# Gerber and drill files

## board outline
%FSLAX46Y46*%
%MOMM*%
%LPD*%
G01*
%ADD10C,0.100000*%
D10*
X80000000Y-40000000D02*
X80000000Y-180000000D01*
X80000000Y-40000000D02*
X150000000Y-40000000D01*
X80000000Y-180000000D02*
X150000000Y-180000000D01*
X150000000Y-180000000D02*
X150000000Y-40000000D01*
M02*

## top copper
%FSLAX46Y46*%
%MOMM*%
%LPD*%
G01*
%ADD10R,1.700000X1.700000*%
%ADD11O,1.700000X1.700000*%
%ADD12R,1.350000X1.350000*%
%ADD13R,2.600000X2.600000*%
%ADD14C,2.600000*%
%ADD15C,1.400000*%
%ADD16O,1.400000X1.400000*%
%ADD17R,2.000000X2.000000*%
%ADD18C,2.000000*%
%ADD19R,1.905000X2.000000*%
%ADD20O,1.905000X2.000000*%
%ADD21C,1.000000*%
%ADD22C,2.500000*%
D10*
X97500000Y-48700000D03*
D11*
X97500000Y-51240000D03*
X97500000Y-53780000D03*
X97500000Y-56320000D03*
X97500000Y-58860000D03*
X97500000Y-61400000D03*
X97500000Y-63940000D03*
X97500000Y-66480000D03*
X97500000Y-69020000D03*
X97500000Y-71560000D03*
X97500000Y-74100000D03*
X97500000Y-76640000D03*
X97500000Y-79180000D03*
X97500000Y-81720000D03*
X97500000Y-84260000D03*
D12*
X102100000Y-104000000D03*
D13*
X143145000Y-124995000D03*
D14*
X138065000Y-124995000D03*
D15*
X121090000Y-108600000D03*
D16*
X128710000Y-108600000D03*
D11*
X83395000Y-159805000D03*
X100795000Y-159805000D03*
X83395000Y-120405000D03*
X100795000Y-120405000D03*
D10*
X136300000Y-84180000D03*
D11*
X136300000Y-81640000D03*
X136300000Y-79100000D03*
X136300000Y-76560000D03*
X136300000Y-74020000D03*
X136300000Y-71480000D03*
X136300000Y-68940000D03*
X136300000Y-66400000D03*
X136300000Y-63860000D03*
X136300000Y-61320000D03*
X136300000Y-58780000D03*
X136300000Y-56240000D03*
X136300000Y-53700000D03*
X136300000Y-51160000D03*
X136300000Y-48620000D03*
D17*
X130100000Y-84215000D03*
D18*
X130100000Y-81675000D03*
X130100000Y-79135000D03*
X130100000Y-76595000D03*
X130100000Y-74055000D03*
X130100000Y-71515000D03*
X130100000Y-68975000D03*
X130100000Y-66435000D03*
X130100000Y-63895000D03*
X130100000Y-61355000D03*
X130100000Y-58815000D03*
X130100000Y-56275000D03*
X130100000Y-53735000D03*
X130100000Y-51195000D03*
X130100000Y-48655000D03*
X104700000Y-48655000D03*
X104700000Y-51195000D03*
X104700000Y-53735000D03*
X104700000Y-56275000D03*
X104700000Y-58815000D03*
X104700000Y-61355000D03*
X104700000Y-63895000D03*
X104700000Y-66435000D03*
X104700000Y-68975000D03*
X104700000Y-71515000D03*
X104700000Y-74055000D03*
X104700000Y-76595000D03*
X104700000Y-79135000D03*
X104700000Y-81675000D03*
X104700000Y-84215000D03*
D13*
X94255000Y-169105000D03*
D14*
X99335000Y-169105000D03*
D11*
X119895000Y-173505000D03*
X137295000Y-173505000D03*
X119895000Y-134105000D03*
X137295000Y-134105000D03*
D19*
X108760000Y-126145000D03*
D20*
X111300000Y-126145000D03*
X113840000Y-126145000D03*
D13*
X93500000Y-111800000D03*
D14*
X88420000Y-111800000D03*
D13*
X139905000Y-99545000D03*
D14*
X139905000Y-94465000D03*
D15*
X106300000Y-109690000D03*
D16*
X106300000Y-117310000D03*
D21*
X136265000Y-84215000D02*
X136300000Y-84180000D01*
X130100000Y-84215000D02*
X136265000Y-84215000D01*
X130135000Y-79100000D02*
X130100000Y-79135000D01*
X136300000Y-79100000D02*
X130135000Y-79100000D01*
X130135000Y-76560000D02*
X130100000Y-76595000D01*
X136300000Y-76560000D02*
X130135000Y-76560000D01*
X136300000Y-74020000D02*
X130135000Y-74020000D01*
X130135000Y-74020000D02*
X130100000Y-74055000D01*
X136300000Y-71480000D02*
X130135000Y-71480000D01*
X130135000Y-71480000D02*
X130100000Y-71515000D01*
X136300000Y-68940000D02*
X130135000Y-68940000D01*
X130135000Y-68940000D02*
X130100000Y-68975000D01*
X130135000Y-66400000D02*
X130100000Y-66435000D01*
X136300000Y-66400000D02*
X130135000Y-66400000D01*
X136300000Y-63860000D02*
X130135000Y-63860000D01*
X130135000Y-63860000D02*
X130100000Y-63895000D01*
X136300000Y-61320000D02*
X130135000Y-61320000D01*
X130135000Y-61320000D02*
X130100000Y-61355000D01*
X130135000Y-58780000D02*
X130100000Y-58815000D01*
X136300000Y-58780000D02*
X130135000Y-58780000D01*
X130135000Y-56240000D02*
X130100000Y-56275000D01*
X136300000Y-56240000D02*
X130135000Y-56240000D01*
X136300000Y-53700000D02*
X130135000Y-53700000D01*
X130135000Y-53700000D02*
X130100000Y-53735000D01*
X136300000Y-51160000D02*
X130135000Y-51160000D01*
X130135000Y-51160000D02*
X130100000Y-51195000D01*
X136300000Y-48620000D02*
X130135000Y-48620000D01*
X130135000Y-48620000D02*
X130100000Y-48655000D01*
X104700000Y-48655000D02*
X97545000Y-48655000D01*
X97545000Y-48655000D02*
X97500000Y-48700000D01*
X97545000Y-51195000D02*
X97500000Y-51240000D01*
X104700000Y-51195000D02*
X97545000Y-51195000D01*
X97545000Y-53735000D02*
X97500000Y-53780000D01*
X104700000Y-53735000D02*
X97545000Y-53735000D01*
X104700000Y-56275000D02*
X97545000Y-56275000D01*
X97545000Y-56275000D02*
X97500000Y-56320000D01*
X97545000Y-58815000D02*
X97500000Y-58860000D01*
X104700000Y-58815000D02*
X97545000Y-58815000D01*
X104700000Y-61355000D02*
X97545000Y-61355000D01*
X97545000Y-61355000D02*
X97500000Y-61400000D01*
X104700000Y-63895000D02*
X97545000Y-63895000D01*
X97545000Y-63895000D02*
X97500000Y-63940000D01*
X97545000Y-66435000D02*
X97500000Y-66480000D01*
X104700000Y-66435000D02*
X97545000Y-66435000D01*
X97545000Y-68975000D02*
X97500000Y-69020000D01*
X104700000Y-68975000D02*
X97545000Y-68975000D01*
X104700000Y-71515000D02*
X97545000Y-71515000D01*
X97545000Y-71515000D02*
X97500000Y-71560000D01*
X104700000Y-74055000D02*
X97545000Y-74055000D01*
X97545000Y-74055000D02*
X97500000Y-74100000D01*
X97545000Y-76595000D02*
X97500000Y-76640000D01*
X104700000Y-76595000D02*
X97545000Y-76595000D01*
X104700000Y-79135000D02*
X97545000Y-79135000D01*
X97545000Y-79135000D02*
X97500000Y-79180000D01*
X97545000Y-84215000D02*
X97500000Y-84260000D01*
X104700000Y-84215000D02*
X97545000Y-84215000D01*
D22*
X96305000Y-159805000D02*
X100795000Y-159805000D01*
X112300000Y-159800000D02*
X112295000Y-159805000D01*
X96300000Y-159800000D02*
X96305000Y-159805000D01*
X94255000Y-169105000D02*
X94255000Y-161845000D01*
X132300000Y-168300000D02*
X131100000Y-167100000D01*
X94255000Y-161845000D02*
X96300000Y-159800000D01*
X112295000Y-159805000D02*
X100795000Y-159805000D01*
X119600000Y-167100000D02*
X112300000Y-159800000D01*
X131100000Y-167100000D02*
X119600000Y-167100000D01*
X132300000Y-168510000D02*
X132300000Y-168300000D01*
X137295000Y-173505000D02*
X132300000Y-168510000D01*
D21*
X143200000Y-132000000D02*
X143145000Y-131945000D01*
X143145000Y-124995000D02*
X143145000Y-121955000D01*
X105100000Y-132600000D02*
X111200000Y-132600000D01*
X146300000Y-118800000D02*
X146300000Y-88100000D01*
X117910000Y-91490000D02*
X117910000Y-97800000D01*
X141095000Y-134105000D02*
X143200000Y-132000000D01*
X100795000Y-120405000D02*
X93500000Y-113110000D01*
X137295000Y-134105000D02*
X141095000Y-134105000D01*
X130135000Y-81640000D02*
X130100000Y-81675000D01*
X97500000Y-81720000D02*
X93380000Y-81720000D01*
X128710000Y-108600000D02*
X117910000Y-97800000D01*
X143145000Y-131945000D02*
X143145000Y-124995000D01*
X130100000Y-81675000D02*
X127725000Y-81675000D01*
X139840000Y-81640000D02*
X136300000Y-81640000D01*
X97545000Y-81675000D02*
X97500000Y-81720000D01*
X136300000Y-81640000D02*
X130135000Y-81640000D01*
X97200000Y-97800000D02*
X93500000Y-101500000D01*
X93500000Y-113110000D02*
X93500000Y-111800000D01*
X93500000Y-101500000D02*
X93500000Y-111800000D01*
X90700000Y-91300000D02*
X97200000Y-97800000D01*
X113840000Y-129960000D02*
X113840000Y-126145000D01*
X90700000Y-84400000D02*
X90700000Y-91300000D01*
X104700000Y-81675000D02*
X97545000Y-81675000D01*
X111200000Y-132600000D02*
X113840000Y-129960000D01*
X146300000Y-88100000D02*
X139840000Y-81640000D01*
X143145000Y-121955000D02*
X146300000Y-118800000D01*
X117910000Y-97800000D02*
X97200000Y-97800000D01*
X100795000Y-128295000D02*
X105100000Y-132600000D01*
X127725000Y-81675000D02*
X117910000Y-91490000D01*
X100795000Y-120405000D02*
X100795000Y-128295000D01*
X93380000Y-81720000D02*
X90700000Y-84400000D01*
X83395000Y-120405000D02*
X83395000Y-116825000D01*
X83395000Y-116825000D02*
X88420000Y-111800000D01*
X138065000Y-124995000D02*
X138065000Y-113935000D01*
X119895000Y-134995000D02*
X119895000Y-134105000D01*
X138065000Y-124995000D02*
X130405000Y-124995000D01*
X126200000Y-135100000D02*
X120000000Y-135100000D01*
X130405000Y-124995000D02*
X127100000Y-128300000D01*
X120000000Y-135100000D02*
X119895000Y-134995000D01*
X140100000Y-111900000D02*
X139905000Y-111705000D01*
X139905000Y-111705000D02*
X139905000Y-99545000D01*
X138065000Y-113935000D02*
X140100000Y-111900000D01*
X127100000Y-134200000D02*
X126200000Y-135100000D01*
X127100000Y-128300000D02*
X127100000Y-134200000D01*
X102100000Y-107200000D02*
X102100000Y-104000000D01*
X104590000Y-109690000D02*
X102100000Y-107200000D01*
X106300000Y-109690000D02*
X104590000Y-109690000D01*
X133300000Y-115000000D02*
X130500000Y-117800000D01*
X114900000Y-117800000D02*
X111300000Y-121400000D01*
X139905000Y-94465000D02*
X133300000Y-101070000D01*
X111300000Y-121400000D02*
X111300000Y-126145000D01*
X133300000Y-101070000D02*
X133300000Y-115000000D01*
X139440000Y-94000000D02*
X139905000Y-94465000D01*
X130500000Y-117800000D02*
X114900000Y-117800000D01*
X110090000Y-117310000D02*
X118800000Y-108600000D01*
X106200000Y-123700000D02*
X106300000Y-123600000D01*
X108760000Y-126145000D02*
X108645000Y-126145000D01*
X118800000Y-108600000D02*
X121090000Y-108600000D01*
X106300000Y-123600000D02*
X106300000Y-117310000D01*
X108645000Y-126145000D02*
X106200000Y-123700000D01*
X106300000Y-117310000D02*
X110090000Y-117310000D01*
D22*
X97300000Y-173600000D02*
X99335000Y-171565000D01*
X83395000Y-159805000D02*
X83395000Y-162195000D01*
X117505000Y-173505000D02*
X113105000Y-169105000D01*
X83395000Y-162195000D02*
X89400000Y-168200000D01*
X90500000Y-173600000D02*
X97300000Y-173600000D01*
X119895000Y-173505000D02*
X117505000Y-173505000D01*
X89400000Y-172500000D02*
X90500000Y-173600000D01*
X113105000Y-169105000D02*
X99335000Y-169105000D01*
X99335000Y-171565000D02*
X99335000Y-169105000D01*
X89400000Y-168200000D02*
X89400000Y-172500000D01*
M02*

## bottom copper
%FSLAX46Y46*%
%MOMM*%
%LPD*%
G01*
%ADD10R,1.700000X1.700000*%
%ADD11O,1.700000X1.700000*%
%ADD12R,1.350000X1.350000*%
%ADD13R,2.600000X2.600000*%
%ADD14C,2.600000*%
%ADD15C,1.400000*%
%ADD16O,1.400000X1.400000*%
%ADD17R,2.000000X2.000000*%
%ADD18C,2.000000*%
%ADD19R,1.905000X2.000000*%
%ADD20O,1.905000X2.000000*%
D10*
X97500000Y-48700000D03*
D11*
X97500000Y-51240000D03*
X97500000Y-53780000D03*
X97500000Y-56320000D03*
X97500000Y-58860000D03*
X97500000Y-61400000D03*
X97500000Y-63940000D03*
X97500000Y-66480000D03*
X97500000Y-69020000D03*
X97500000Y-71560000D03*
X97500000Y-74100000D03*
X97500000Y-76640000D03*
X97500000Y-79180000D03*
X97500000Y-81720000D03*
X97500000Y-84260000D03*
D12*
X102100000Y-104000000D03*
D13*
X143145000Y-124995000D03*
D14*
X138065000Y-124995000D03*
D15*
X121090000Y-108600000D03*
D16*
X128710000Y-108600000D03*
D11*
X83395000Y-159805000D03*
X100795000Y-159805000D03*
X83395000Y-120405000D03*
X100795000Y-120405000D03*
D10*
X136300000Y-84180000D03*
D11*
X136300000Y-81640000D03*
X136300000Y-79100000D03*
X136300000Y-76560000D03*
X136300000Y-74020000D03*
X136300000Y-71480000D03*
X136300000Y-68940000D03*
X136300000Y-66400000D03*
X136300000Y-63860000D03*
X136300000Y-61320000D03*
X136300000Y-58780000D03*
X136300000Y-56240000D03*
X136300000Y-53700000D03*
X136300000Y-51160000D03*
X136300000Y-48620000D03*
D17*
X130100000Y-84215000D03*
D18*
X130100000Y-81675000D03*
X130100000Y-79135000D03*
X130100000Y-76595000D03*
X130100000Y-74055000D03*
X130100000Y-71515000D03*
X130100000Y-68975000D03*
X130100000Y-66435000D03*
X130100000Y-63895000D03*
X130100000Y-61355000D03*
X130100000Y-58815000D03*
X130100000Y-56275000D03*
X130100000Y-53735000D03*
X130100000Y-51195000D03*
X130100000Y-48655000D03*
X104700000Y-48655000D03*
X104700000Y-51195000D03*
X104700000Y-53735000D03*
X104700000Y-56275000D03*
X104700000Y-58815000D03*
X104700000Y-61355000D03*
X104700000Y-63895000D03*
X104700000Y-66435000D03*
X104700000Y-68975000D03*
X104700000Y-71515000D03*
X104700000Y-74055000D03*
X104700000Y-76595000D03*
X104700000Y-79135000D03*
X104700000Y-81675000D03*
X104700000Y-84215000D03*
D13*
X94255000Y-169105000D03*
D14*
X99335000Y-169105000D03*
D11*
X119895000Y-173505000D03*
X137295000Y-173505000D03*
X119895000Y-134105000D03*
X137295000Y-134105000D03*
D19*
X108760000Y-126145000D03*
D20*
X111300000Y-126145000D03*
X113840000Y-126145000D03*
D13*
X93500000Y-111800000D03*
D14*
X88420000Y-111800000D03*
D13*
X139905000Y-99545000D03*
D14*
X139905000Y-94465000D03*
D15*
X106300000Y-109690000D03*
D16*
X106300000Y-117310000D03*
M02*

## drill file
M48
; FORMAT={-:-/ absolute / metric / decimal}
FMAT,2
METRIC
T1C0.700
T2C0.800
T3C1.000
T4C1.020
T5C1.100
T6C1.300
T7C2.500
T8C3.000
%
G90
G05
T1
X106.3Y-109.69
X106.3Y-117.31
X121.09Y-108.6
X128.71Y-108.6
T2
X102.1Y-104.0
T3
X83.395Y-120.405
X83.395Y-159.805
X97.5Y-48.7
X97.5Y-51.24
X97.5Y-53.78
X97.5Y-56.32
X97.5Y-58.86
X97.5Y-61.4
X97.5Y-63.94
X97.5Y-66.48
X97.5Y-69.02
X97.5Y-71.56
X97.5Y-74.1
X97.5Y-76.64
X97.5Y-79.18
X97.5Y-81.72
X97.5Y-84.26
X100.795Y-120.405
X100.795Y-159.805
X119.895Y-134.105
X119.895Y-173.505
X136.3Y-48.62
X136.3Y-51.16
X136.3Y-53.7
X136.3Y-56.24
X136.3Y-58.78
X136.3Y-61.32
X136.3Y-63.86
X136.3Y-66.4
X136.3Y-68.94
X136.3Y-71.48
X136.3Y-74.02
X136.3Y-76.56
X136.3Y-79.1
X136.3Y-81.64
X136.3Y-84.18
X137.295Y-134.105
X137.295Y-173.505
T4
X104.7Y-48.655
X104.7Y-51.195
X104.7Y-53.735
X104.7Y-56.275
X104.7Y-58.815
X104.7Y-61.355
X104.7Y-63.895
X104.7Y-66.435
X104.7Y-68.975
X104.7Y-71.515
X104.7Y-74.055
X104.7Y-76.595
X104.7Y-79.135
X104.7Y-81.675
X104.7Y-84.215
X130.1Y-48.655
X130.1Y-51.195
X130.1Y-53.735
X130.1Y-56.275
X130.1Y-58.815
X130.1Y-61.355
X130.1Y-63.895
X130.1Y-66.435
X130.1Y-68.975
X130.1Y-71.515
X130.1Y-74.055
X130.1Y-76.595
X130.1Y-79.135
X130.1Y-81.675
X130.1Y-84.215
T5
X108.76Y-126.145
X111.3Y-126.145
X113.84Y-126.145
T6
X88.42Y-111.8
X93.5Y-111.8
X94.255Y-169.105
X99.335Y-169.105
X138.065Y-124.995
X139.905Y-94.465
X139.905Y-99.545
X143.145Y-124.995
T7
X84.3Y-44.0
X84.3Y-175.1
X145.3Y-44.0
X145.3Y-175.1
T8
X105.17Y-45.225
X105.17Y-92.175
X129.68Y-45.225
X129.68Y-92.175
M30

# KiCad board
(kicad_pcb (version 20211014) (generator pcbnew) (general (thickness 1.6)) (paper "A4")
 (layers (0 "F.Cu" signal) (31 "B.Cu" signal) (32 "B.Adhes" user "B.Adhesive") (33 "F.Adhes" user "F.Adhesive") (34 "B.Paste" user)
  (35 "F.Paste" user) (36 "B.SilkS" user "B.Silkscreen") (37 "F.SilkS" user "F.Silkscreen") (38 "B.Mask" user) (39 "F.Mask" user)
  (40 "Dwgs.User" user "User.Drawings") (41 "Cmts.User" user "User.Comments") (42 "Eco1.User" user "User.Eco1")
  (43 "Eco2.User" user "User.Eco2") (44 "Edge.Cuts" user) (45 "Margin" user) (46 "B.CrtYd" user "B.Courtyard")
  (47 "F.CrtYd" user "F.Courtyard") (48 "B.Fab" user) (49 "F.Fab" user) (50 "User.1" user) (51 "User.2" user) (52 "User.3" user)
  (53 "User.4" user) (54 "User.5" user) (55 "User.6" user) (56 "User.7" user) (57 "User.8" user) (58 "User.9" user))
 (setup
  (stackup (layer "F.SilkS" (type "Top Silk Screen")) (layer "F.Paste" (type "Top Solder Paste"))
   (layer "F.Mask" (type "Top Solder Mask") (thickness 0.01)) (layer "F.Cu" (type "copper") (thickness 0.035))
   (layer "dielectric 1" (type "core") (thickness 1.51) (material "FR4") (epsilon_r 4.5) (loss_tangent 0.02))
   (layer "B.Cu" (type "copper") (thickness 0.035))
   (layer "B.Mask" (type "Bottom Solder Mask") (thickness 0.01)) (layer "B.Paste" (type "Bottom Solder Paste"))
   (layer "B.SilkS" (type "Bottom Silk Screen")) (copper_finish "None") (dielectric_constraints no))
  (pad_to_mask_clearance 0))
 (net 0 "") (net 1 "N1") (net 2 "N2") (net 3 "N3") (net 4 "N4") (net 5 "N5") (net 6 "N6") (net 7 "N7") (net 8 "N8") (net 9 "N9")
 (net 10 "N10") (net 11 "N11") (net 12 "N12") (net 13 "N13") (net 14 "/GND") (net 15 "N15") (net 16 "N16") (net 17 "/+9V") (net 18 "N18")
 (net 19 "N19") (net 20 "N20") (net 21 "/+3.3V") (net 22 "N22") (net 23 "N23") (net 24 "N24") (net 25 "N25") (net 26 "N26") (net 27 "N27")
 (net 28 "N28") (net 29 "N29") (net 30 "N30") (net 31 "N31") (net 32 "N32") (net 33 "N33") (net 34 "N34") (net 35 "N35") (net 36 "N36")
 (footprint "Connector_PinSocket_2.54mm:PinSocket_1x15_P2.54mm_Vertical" (layer "F.Cu") (at 97.5 48.7)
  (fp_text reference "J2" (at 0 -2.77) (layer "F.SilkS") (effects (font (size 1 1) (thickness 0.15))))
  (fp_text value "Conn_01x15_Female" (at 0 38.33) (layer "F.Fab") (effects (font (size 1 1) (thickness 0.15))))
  (pad "1" thru_hole rect (at 0 0) (size 1.7 1.7) (drill 1) (layers *.Cu *.Mask) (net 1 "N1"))
  (pad "2" thru_hole oval (at 0 2.54) (size 1.7 1.7) (drill 1) (layers *.Cu *.Mask) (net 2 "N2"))
  (pad "3" thru_hole oval (at 0 5.08) (size 1.7 1.7) (drill 1) (layers *.Cu *.Mask) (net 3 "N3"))
  (pad "4" thru_hole oval (at 0 7.62) (size 1.7 1.7) (drill 1) (layers *.Cu *.Mask) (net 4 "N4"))
  (pad "5" thru_hole oval (at 0 10.16) (size 1.7 1.7) (drill 1) (layers *.Cu *.Mask) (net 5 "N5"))
  (pad "6" thru_hole oval (at 0 12.7) (size 1.7 1.7) (drill 1) (layers *.Cu *.Mask) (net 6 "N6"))
  (pad "7" thru_hole oval (at 0 15.24) (size 1.7 1.7) (drill 1) (layers *.Cu *.Mask) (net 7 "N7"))
  (pad "8" thru_hole oval (at 0 17.78) (size 1.7 1.7) (drill 1) (layers *.Cu *.Mask) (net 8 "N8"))
  (pad "9" thru_hole oval (at 0 20.32) (size 1.7 1.7) (drill 1) (layers *.Cu *.Mask) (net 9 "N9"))
  (pad "10" thru_hole oval (at 0 22.86) (size 1.7 1.7) (drill 1) (layers *.Cu *.Mask) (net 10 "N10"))
  (pad "11" thru_hole oval (at 0 25.4) (size 1.7 1.7) (drill 1) (layers *.Cu *.Mask) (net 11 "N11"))
  (pad "12" thru_hole oval (at 0 27.94) (size 1.7 1.7) (drill 1) (layers *.Cu *.Mask) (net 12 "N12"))
  (pad "13" thru_hole oval (at 0 30.48) (size 1.7 1.7) (drill 1) (layers *.Cu *.Mask) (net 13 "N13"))
  (pad "14" thru_hole oval (at 0 33.02) (size 1.7 1.7) (drill 1) (layers *.Cu *.Mask) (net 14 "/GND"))
  (pad "15" thru_hole oval (at 0 35.56) (size 1.7 1.7) (drill 1) (layers *.Cu *.Mask) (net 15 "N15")))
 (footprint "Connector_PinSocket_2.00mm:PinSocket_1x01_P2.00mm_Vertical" (layer "F.Cu") (at 102.1 104)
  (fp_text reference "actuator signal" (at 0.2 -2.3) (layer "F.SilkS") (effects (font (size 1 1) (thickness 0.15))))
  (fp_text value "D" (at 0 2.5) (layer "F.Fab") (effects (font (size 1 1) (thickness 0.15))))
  (pad "1" thru_hole rect (at 0 0) (size 1.35 1.35) (drill 0.8) (layers *.Cu *.Mask) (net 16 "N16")))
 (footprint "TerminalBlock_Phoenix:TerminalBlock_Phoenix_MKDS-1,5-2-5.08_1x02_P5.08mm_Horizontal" (layer "F.Cu") (at 143.145 124.995 180)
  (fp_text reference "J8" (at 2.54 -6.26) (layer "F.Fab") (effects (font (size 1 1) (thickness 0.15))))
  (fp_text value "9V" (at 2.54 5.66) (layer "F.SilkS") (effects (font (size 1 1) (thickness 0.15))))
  (pad "1" thru_hole rect (at 0 0 180) (size 2.6 2.6) (drill 1.3) (layers *.Cu *.Mask) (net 14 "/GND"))
  (pad "2" thru_hole circle (at 5.08 0 180) (size 2.6 2.6) (drill 1.3) (layers *.Cu *.Mask) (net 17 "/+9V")))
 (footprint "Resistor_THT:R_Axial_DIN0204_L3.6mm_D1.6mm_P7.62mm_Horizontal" (layer "F.Cu") (at 121.09 108.6)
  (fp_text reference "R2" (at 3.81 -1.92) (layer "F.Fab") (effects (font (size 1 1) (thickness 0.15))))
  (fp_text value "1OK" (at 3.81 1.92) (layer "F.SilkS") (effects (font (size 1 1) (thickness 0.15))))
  (pad "1" thru_hole circle (at 0 0) (size 1.4 1.4) (drill 0.7) (layers *.Cu *.Mask) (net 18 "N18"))
  (pad "2" thru_hole oval (at 7.62 0) (size 1.4 1.4) (drill 0.7) (layers *.Cu *.Mask) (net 14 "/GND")))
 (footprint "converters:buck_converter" (layer "F.Cu") (at 81.595 161.805 90)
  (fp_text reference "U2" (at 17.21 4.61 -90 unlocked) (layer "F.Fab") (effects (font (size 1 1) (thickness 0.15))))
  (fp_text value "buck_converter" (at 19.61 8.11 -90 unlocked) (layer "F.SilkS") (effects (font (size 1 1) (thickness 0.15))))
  (pad "1" thru_hole oval (at 2 1.8 90) (size 1.7 1.7) (drill 1) (layers *.Cu *.Mask) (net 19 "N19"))
  (pad "2" thru_hole oval (at 2 19.2 90) (size 1.7 1.7) (drill 1) (layers *.Cu *.Mask) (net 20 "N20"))
  (pad "3" thru_hole oval (at 41.4 1.8 90) (size 1.7 1.7) (drill 1) (layers *.Cu *.Mask) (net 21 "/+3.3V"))
  (pad "4" thru_hole oval (at 41.4 19.2 90) (size 1.7 1.7) (drill 1) (layers *.Cu *.Mask) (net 14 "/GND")))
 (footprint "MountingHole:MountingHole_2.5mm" (layer "F.Cu") (at 145.3 44)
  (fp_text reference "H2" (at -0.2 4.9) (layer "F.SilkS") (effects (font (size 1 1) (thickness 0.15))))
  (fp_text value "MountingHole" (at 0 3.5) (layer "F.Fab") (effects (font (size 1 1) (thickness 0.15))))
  (pad "" np_thru_hole circle (at 0 0) (size 2.5 2.5) (drill 2.5) (layers *.Cu *.Mask)))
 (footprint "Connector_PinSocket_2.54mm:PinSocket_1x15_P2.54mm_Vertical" (layer "F.Cu") (at 136.3 84.18 180)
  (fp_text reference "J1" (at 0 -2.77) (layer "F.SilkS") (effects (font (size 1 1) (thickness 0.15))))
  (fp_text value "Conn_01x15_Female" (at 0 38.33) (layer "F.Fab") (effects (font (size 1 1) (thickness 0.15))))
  (pad "1" thru_hole rect (at 0 0 180) (size 1.7 1.7) (drill 1) (layers *.Cu *.Mask) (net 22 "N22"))
  (pad "2" thru_hole oval (at 0 2.54 180) (size 1.7 1.7) (drill 1) (layers *.Cu *.Mask) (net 14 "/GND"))
  (pad "3" thru_hole oval (at 0 5.08 180) (size 1.7 1.7) (drill 1) (layers *.Cu *.Mask) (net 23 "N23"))
  (pad "4" thru_hole oval (at 0 7.62 180) (size 1.7 1.7) (drill 1) (layers *.Cu *.Mask) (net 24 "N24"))
  (pad "5" thru_hole oval (at 0 10.16 180) (size 1.7 1.7) (drill 1) (layers *.Cu *.Mask) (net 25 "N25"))
  (pad "6" thru_hole oval (at 0 12.7 180) (size 1.7 1.7) (drill 1) (layers *.Cu *.Mask) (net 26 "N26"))
  (pad "7" thru_hole oval (at 0 15.24 180) (size 1.7 1.7) (drill 1) (layers *.Cu *.Mask) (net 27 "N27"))
  (pad "8" thru_hole oval (at 0 17.78 180) (size 1.7 1.7) (drill 1) (layers *.Cu *.Mask) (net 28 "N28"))
  (pad "9" thru_hole oval (at 0 20.32 180) (size 1.7 1.7) (drill 1) (layers *.Cu *.Mask) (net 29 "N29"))
  (pad "10" thru_hole oval (at 0 22.86 180) (size 1.7 1.7) (drill 1) (layers *.Cu *.Mask) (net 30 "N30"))
  (pad "11" thru_hole oval (at 0 25.4 180) (size 1.7 1.7) (drill 1) (layers *.Cu *.Mask) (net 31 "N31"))
  (pad "12" thru_hole oval (at 0 27.94 180) (size 1.7 1.7) (drill 1) (layers *.Cu *.Mask) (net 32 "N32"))
  (pad "13" thru_hole oval (at 0 30.48 180) (size 1.7 1.7) (drill 1) (layers *.Cu *.Mask) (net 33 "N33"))
  (pad "14" thru_hole oval (at 0 33.02 180) (size 1.7 1.7) (drill 1) (layers *.Cu *.Mask) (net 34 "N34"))
  (pad "15" thru_hole oval (at 0 35.56 180) (size 1.7 1.7) (drill 1) (layers *.Cu *.Mask) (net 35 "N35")))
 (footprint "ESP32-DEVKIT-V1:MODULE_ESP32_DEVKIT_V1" (layer "F.Cu") (at 117.4 68.7 180)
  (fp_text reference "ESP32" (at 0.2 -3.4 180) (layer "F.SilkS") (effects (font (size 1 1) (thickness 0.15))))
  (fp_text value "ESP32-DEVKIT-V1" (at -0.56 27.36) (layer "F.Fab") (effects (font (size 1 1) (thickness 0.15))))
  (pad "" np_thru_hole circle locked (at -12.28 23.475 180) (size 3 3) (drill 3) (layers *.Cu *.Mask))
  (pad "" np_thru_hole circle locked (at -12.28 -23.475 180) (size 3 3) (drill 3) (layers *.Cu *.Mask))
  (pad "" np_thru_hole circle locked (at 12.23 23.475 180) (size 3 3) (drill 3) (layers *.Cu *.Mask))
  (pad "" np_thru_hole circle locked (at 12.23 -23.475 180) (size 3 3) (drill 3) (layers *.Cu *.Mask))
  (pad "1" thru_hole rect locked (at -12.7 -15.515 180) (size 2 2) (drill 1.02) (layers *.Cu *.Mask) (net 22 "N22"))
  (pad "2" thru_hole circle locked (at -12.7 -12.975 180) (size 2 2) (drill 1.02) (layers *.Cu *.Mask) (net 14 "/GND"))
  (pad "3" thru_hole circle locked (at -12.7 -10.435 180) (size 2 2) (drill 1.02) (layers *.Cu *.Mask) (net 23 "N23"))
  (pad "4" thru_hole circle locked (at -12.7 -7.895 180) (size 2 2) (drill 1.02) (layers *.Cu *.Mask) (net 24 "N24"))
  (pad "5" thru_hole circle locked (at -12.7 -5.355 180) (size 2 2) (drill 1.02) (layers *.Cu *.Mask) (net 25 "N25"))
  (pad "6" thru_hole circle locked (at -12.7 -2.815 180) (size 2 2) (drill 1.02) (layers *.Cu *.Mask) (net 26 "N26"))
  (pad "7" thru_hole circle locked (at -12.7 -0.275 180) (size 2 2) (drill 1.02) (layers *.Cu *.Mask) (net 27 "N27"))
  (pad "8" thru_hole circle locked (at -12.7 2.265 180) (size 2 2) (drill 1.02) (layers *.Cu *.Mask) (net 28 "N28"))
  (pad "9" thru_hole circle locked (at -12.7 4.805 180) (size 2 2) (drill 1.02) (layers *.Cu *.Mask) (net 29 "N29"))
  (pad "10" thru_hole circle locked (at -12.7 7.345 180) (size 2 2) (drill 1.02) (layers *.Cu *.Mask) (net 30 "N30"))
  (pad "11" thru_hole circle locked (at -12.7 9.885 180) (size 2 2) (drill 1.02) (layers *.Cu *.Mask) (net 31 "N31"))
  (pad "12" thru_hole circle locked (at -12.7 12.425 180) (size 2 2) (drill 1.02) (layers *.Cu *.Mask) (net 32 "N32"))
  (pad "13" thru_hole circle locked (at -12.7 14.965 180) (size 2 2) (drill 1.02) (layers *.Cu *.Mask) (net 33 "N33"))
  (pad "14" thru_hole circle locked (at -12.7 17.505 180) (size 2 2) (drill 1.02) (layers *.Cu *.Mask) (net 34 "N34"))
  (pad "15" thru_hole circle locked (at -12.7 20.045 180) (size 2 2) (drill 1.02) (layers *.Cu *.Mask) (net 35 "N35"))
  (pad "16" thru_hole circle locked (at 12.7 20.045 180) (size 2 2) (drill 1.02) (layers *.Cu *.Mask) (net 1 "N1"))
  (pad "17" thru_hole circle locked (at 12.7 17.505 180) (size 2 2) (drill 1.02) (layers *.Cu *.Mask) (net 2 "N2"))
  (pad "18" thru_hole circle locked (at 12.7 14.965 180) (size 2 2) (drill 1.02) (layers *.Cu *.Mask) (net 3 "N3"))
  (pad "19" thru_hole circle locked (at 12.7 12.425 180) (size 2 2) (drill 1.02) (layers *.Cu *.Mask) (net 4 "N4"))
  (pad "20" thru_hole circle locked (at 12.7 9.885 180) (size 2 2) (drill 1.02) (layers *.Cu *.Mask) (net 5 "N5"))
  (pad "21" thru_hole circle locked (at 12.7 7.345 180) (size 2 2) (drill 1.02) (layers *.Cu *.Mask) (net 6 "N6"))
  (pad "22" thru_hole circle locked (at 12.7 4.805 180) (size 2 2) (drill 1.02) (layers *.Cu *.Mask) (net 7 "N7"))
  (pad "23" thru_hole circle locked (at 12.7 2.265 180) (size 2 2) (drill 1.02) (layers *.Cu *.Mask) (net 8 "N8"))
  (pad "24" thru_hole circle locked (at 12.7 -0.275 180) (size 2 2) (drill 1.02) (layers *.Cu *.Mask) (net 9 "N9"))
  (pad "25" thru_hole circle locked (at 12.7 -2.815 180) (size 2 2) (drill 1.02) (layers *.Cu *.Mask) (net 10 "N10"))
  (pad "26" thru_hole circle locked (at 12.7 -5.355 180) (size 2 2) (drill 1.02) (layers *.Cu *.Mask) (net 11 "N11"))
  (pad "27" thru_hole circle locked (at 12.7 -7.895 180) (size 2 2) (drill 1.02) (layers *.Cu *.Mask) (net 12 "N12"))
  (pad "28" thru_hole circle locked (at 12.7 -10.435 180) (size 2 2) (drill 1.02) (layers *.Cu *.Mask) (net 13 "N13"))
  (pad "29" thru_hole circle locked (at 12.7 -12.975 180) (size 2 2) (drill 1.02) (layers *.Cu *.Mask) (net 14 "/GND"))
  (pad "30" thru_hole circle locked (at 12.7 -15.515 180) (size 2 2) (drill 1.02) (layers *.Cu *.Mask) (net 15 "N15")))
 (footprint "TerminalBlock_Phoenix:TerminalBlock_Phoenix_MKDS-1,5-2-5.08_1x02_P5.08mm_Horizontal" (layer "F.Cu") (at 94.255 169.105)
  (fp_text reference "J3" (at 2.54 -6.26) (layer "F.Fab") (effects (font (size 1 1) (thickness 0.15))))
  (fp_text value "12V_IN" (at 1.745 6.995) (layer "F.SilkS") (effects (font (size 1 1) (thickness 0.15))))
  (pad "1" thru_hole rect (at 0 0) (size 2.6 2.6) (drill 1.3) (layers *.Cu *.Mask) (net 20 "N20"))
  (pad "2" thru_hole circle (at 5.08 0) (size 2.6 2.6) (drill 1.3) (layers *.Cu *.Mask) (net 19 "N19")))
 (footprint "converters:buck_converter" (layer "F.Cu") (at 118.095 175.505 90)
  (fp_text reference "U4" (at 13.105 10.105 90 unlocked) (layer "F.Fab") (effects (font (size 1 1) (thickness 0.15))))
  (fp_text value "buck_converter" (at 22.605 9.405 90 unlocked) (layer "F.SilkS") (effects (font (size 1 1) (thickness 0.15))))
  (pad "1" thru_hole oval (at 2 1.8 90) (size 1.7 1.7) (drill 1) (layers *.Cu *.Mask) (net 19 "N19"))
  (pad "2" thru_hole oval (at 2 19.2 90) (size 1.7 1.7) (drill 1) (layers *.Cu *.Mask) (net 20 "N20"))
  (pad "3" thru_hole oval (at 41.4 1.8 90) (size 1.7 1.7) (drill 1) (layers *.Cu *.Mask) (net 17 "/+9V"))
  (pad "4" thru_hole oval (at 41.4 19.2 90) (size 1.7 1.7) (drill 1) (layers *.Cu *.Mask) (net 14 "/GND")))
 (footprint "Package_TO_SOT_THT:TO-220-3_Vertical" (layer "F.Cu") (at 108.76 126.145)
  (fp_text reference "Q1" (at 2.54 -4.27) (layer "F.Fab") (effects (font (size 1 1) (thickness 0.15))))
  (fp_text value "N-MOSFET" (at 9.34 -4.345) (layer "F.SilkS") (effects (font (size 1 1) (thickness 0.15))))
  (pad "1" thru_hole rect (at 0 0) (size 1.905 2) (drill 1.1) (layers *.Cu *.Mask) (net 18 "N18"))
  (pad "2" thru_hole oval (at 2.54 0) (size 1.905 2) (drill 1.1) (layers *.Cu *.Mask) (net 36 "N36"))
  (pad "3" thru_hole oval (at 5.08 0) (size 1.905 2) (drill 1.1) (layers *.Cu *.Mask) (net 14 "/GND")))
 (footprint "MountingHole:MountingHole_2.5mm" (layer "F.Cu") (at 145.3 175.1)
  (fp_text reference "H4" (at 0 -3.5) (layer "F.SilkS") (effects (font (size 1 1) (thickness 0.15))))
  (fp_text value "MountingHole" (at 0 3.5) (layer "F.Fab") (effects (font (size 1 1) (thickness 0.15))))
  (pad "" np_thru_hole circle (at 0 0) (size 2.5 2.5) (drill 2.5) (layers *.Cu *.Mask)))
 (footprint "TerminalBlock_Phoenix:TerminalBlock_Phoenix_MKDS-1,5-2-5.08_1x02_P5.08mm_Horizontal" (layer "F.Cu") (at 93.5 111.8 180)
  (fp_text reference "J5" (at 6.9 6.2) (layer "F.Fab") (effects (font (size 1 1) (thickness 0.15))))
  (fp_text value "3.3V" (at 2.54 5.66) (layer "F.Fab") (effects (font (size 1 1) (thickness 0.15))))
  (pad "1" thru_hole rect (at 0 0 180) (size 2.6 2.6) (drill 1.3) (layers *.Cu *.Mask) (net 14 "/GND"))
  (pad "2" thru_hole circle (at 5.08 0 180) (size 2.6 2.6) (drill 1.3) (layers *.Cu *.Mask) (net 21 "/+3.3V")))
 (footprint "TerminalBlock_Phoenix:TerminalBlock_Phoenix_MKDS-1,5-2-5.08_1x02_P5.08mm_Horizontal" (layer "F.Cu") (at 139.905 99.545 90)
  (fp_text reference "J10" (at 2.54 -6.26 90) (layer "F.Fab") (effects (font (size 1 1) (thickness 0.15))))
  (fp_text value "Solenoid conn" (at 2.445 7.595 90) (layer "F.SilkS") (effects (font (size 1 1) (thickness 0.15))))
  (pad "1" thru_hole rect (at 0 0 90) (size 2.6 2.6) (drill 1.3) (layers *.Cu *.Mask) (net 17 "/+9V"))
  (pad "2" thru_hole circle (at 5.08 0 90) (size 2.6 2.6) (drill 1.3) (layers *.Cu *.Mask) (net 36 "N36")))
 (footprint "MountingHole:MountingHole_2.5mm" (layer "F.Cu") (at 84.3 44)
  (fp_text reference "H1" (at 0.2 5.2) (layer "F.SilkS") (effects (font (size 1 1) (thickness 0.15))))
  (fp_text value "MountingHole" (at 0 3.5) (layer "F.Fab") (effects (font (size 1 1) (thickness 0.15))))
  (pad "" np_thru_hole circle (at 0 0) (size 2.5 2.5) (drill 2.5) (layers *.Cu *.Mask)))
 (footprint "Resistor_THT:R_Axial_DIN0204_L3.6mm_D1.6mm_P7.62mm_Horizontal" (layer "F.Cu") (at 106.3 109.69 -90)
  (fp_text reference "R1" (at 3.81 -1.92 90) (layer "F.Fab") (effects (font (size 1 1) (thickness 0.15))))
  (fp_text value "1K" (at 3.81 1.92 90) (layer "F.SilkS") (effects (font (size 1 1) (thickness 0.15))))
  (pad "1" thru_hole circle (at 0 0 270) (size 1.4 1.4) (drill 0.7) (layers *.Cu *.Mask) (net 16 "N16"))
  (pad "2" thru_hole oval (at 7.62 0 270) (size 1.4 1.4) (drill 0.7) (layers *.Cu *.Mask) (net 18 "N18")))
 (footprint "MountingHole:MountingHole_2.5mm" (layer "F.Cu") (at 84.3 175.1)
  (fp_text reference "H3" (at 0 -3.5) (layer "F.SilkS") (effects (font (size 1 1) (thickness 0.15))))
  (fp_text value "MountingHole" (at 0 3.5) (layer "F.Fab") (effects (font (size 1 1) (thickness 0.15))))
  (pad "" np_thru_hole circle (at 0 0) (size 2.5 2.5) (drill 2.5) (layers *.Cu *.Mask)))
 (gr_line (start 80 40) (end 80 180) (layer "Edge.Cuts") (width 0.1))
 (gr_line (start 80 40) (end 150 40) (layer "Edge.Cuts") (width 0.1))
 (gr_line (start 80 180) (end 150 180) (layer "Edge.Cuts") (width 0.1))
 (gr_line (start 150 180) (end 150 40) (layer "Edge.Cuts") (width 0.1))
 (segment (start 136.265 84.215) (end 136.3 84.18) (width 1) (layer "F.Cu") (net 22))
 (segment (start 130.1 84.215) (end 136.265 84.215) (width 1) (layer "F.Cu") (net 22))
 (segment (start 130.135 79.1) (end 130.1 79.135) (width 1) (layer "F.Cu") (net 23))
 (segment (start 136.3 79.1) (end 130.135 79.1) (width 1) (layer "F.Cu") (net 23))
 (segment (start 130.135 76.56) (end 130.1 76.595) (width 1) (layer "F.Cu") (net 24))
 (segment (start 136.3 76.56) (end 130.135 76.56) (width 1) (layer "F.Cu") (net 24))
 (segment (start 136.3 74.02) (end 130.135 74.02) (width 1) (layer "F.Cu") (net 25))
 (segment (start 130.135 74.02) (end 130.1 74.055) (width 1) (layer "F.Cu") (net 25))
 (segment (start 136.3 71.48) (end 130.135 71.48) (width 1) (layer "F.Cu") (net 26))
 (segment (start 130.135 71.48) (end 130.1 71.515) (width 1) (layer "F.Cu") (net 26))
 (segment (start 136.3 68.94) (end 130.135 68.94) (width 1) (layer "F.Cu") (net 27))
 (segment (start 130.135 68.94) (end 130.1 68.975) (width 1) (layer "F.Cu") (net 27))
 (segment (start 130.135 66.4) (end 130.1 66.435) (width 1) (layer "F.Cu") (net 28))
 (segment (start 136.3 66.4) (end 130.135 66.4) (width 1) (layer "F.Cu") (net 28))
 (segment (start 136.3 63.86) (end 130.135 63.86) (width 1) (layer "F.Cu") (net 29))
 (segment (start 130.135 63.86) (end 130.1 63.895) (width 1) (layer "F.Cu") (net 29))
 (segment (start 136.3 61.32) (end 130.135 61.32) (width 1) (layer "F.Cu") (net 30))
 (segment (start 130.135 61.32) (end 130.1 61.355) (width 1) (layer "F.Cu") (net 30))
 (segment (start 130.135 58.78) (end 130.1 58.815) (width 1) (layer "F.Cu") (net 31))
 (segment (start 136.3 58.78) (end 130.135 58.78) (width 1) (layer "F.Cu") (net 31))
 (segment (start 130.135 56.24) (end 130.1 56.275) (width 1) (layer "F.Cu") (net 32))
 (segment (start 136.3 56.24) (end 130.135 56.24) (width 1) (layer "F.Cu") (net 32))
 (segment (start 136.3 53.7) (end 130.135 53.7) (width 1) (layer "F.Cu") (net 33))
 (segment (start 130.135 53.7) (end 130.1 53.735) (width 1) (layer "F.Cu") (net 33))
 (segment (start 136.3 51.16) (end 130.135 51.16) (width 1) (layer "F.Cu") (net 34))
 (segment (start 130.135 51.16) (end 130.1 51.195) (width 1) (layer "F.Cu") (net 34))
 (segment (start 136.3 48.62) (end 130.135 48.62) (width 1) (layer "F.Cu") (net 35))
 (segment (start 130.135 48.62) (end 130.1 48.655) (width 1) (layer "F.Cu") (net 35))
 (segment (start 104.7 48.655) (end 97.545 48.655) (width 1) (layer "F.Cu") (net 1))
 (segment (start 97.545 48.655) (end 97.5 48.7) (width 1) (layer "F.Cu") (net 1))
 (segment (start 97.545 51.195) (end 97.5 51.24) (width 1) (layer "F.Cu") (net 2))
 (segment (start 104.7 51.195) (end 97.545 51.195) (width 1) (layer "F.Cu") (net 2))
 (segment (start 97.545 53.735) (end 97.5 53.78) (width 1) (layer "F.Cu") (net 3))
 (segment (start 104.7 53.735) (end 97.545 53.735) (width 1) (layer "F.Cu") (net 3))
 (segment (start 104.7 56.275) (end 97.545 56.275) (width 1) (layer "F.Cu") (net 4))
 (segment (start 97.545 56.275) (end 97.5 56.32) (width 1) (layer "F.Cu") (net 4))
 (segment (start 97.545 58.815) (end 97.5 58.86) (width 1) (layer "F.Cu") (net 5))
 (segment (start 104.7 58.815) (end 97.545 58.815) (width 1) (layer "F.Cu") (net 5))
 (segment (start 104.7 61.355) (end 97.545 61.355) (width 1) (layer "F.Cu") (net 6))
 (segment (start 97.545 61.355) (end 97.5 61.4) (width 1) (layer "F.Cu") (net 6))
 (segment (start 104.7 63.895) (end 97.545 63.895) (width 1) (layer "F.Cu") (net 7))
 (segment (start 97.545 63.895) (end 97.5 63.94) (width 1) (layer "F.Cu") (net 7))
 (segment (start 97.545 66.435) (end 97.5 66.48) (width 1) (layer "F.Cu") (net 8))
 (segment (start 104.7 66.435) (end 97.545 66.435) (width 1) (layer "F.Cu") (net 8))
 (segment (start 97.545 68.975) (end 97.5 69.02) (width 1) (layer "F.Cu") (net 9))
 (segment (start 104.7 68.975) (end 97.545 68.975) (width 1) (layer "F.Cu") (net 9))
 (segment (start 104.7 71.515) (end 97.545 71.515) (width 1) (layer "F.Cu") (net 10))
 (segment (start 97.545 71.515) (end 97.5 71.56) (width 1) (layer "F.Cu") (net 10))
 (segment (start 104.7 74.055) (end 97.545 74.055) (width 1) (layer "F.Cu") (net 11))
 (segment (start 97.545 74.055) (end 97.5 74.1) (width 1) (layer "F.Cu") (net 11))
 (segment (start 97.545 76.595) (end 97.5 76.64) (width 1) (layer "F.Cu") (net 12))
 (segment (start 104.7 76.595) (end 97.545 76.595) (width 1) (layer "F.Cu") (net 12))
 (segment (start 104.7 79.135) (end 97.545 79.135) (width 1) (layer "F.Cu") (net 13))
 (segment (start 97.545 79.135) (end 97.5 79.18) (width 1) (layer "F.Cu") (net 13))
 (segment (start 97.545 84.215) (end 97.5 84.26) (width 1) (layer "F.Cu") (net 15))
 (segment (start 104.7 84.215) (end 97.545 84.215) (width 1) (layer "F.Cu") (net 15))
 (segment (start 96.305 159.805) (end 100.795 159.805) (width 2.5) (layer "F.Cu") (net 20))
 (segment (start 112.3 159.8) (end 112.295 159.805) (width 2.5) (layer "F.Cu") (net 20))
 (segment (start 96.3 159.8) (end 96.305 159.805) (width 2.5) (layer "F.Cu") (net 20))
 (segment (start 94.255 169.105) (end 94.255 161.845) (width 2.5) (layer "F.Cu") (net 20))
 (segment (start 132.3 168.3) (end 131.1 167.1) (width 2.5) (layer "F.Cu") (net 20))
 (segment (start 94.255 161.845) (end 96.3 159.8) (width 2.5) (layer "F.Cu") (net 20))
 (segment (start 112.295 159.805) (end 100.795 159.805) (width 2.5) (layer "F.Cu") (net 20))
 (segment (start 119.6 167.1) (end 112.3 159.8) (width 2.5) (layer "F.Cu") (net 20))
 (segment (start 131.1 167.1) (end 119.6 167.1) (width 2.5) (layer "F.Cu") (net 20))
 (segment (start 132.3 168.51) (end 132.3 168.3) (width 2.5) (layer "F.Cu") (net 20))
 (segment (start 137.295 173.505) (end 132.3 168.51) (width 2.5) (layer "F.Cu") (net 20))
 (segment (start 143.2 132) (end 143.145 131.945) (width 1) (layer "F.Cu") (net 14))
 (segment (start 143.145 124.995) (end 143.145 121.955) (width 1) (layer "F.Cu") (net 14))
 (segment (start 105.1 132.6) (end 111.2 132.6) (width 1) (layer "F.Cu") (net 14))
 (segment (start 146.3 118.8) (end 146.3 88.1) (width 1) (layer "F.Cu") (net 14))
 (segment (start 117.91 91.49) (end 117.91 97.8) (width 1) (layer "F.Cu") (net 14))
 (segment (start 141.095 134.105) (end 143.2 132) (width 1) (layer "F.Cu") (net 14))
 (segment (start 100.795 120.405) (end 93.5 113.11) (width 1) (layer "F.Cu") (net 14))
 (segment (start 137.295 134.105) (end 141.095 134.105) (width 1) (layer "F.Cu") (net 14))
 (segment (start 130.135 81.64) (end 130.1 81.675) (width 1) (layer "F.Cu") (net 14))
 (segment (start 97.5 81.72) (end 93.38 81.72) (width 1) (layer "F.Cu") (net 14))
 (segment (start 128.71 108.6) (end 117.91 97.8) (width 1) (layer "F.Cu") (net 14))
 (segment (start 143.145 131.945) (end 143.145 124.995) (width 1) (layer "F.Cu") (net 14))
 (segment (start 130.1 81.675) (end 127.725 81.675) (width 1) (layer "F.Cu") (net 14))
 (segment (start 139.84 81.64) (end 136.3 81.64) (width 1) (layer "F.Cu") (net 14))
 (segment (start 97.545 81.675) (end 97.5 81.72) (width 1) (layer "F.Cu") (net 14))
 (segment (start 136.3 81.64) (end 130.135 81.64) (width 1) (layer "F.Cu") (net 14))
 (segment (start 97.2 97.8) (end 93.5 101.5) (width 1) (layer "F.Cu") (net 14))
 (segment (start 93.5 113.11) (end 93.5 111.8) (width 1) (layer "F.Cu") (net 14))
 (segment (start 93.5 101.5) (end 93.5 111.8) (width 1) (layer "F.Cu") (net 14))
 (segment (start 90.7 91.3) (end 97.2 97.8) (width 1) (layer "F.Cu") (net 14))
 (segment (start 113.84 129.96) (end 113.84 126.145) (width 1) (layer "F.Cu") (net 14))
 (segment (start 90.7 84.4) (end 90.7 91.3) (width 1) (layer "F.Cu") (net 14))
 (segment (start 104.7 81.675) (end 97.545 81.675) (width 1) (layer "F.Cu") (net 14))
 (segment (start 111.2 132.6) (end 113.84 129.96) (width 1) (layer "F.Cu") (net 14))
 (segment (start 146.3 88.1) (end 139.84 81.64) (width 1) (layer "F.Cu") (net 14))
 (segment (start 143.145 121.955) (end 146.3 118.8) (width 1) (layer "F.Cu") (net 14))
 (segment (start 117.91 97.8) (end 97.2 97.8) (width 1) (layer "F.Cu") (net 14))
 (segment (start 100.795 128.295) (end 105.1 132.6) (width 1) (layer "F.Cu") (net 14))
 (segment (start 127.725 81.675) (end 117.91 91.49) (width 1) (layer "F.Cu") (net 14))
 (segment (start 100.795 120.405) (end 100.795 128.295) (width 1) (layer "F.Cu") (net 14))
 (segment (start 93.38 81.72) (end 90.7 84.4) (width 1) (layer "F.Cu") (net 14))
 (segment (start 83.395 120.405) (end 83.395 116.825) (width 1) (layer "F.Cu") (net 21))
 (segment (start 83.395 116.825) (end 88.42 111.8) (width 1) (layer "F.Cu") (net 21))
 (segment (start 138.065 124.995) (end 138.065 113.935) (width 1) (layer "F.Cu") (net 17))
 (segment (start 119.895 134.995) (end 119.895 134.105) (width 1) (layer "F.Cu") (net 17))
 (segment (start 138.065 124.995) (end 130.405 124.995) (width 1) (layer "F.Cu") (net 17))
 (segment (start 126.2 135.1) (end 120 135.1) (width 1) (layer "F.Cu") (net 17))
 (segment (start 130.405 124.995) (end 127.1 128.3) (width 1) (layer "F.Cu") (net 17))
 (segment (start 120 135.1) (end 119.895 134.995) (width 1) (layer "F.Cu") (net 17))
 (segment (start 140.1 111.9) (end 139.905 111.705) (width 1) (layer "F.Cu") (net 17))
 (segment (start 139.905 111.705) (end 139.905 99.545) (width 1) (layer "F.Cu") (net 17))
 (segment (start 138.065 113.935) (end 140.1 111.9) (width 1) (layer "F.Cu") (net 17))
 (segment (start 127.1 134.2) (end 126.2 135.1) (width 1) (layer "F.Cu") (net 17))
 (segment (start 127.1 128.3) (end 127.1 134.2) (width 1) (layer "F.Cu") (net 17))
 (segment (start 102.1 107.2) (end 102.1 104) (width 1) (layer "F.Cu") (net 16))
 (segment (start 104.59 109.69) (end 102.1 107.2) (width 1) (layer "F.Cu") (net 16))
 (segment (start 106.3 109.69) (end 104.59 109.69) (width 1) (layer "F.Cu") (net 16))
 (segment (start 133.3 115) (end 130.5 117.8) (width 1) (layer "F.Cu") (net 36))
 (segment (start 114.9 117.8) (end 111.3 121.4) (width 1) (layer "F.Cu") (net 36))
 (segment (start 139.905 94.465) (end 133.3 101.07) (width 1) (layer "F.Cu") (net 36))
 (segment (start 111.3 121.4) (end 111.3 126.145) (width 1) (layer "F.Cu") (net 36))
 (segment (start 133.3 101.07) (end 133.3 115) (width 1) (layer "F.Cu") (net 36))
 (segment (start 139.44 94) (end 139.905 94.465) (width 1) (layer "F.Cu") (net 36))
 (segment (start 130.5 117.8) (end 114.9 117.8) (width 1) (layer "F.Cu") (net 36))
 (segment (start 110.09 117.31) (end 118.8 108.6) (width 1) (layer "F.Cu") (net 18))
 (segment (start 106.2 123.7) (end 106.3 123.6) (width 1) (layer "F.Cu") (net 18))
 (segment (start 108.76 126.145) (end 108.645 126.145) (width 1) (layer "F.Cu") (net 18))
 (segment (start 118.8 108.6) (end 121.09 108.6) (width 1) (layer "F.Cu") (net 18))
 (segment (start 106.3 123.6) (end 106.3 117.31) (width 1) (layer "F.Cu") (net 18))
 (segment (start 108.645 126.145) (end 106.2 123.7) (width 1) (layer "F.Cu") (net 18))
 (segment (start 106.3 117.31) (end 110.09 117.31) (width 1) (layer "F.Cu") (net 18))
 (segment (start 97.3 173.6) (end 99.335 171.565) (width 2.5) (layer "F.Cu") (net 19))
 (segment (start 83.395 159.805) (end 83.395 162.195) (width 2.5) (layer "F.Cu") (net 19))
 (segment (start 117.505 173.505) (end 113.105 169.105) (width 2.5) (layer "F.Cu") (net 19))
 (segment (start 83.395 162.195) (end 89.4 168.2) (width 2.5) (layer "F.Cu") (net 19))
 (segment (start 90.5 173.6) (end 97.3 173.6) (width 2.5) (layer "F.Cu") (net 19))
 (segment (start 119.895 173.505) (end 117.505 173.505) (width 2.5) (layer "F.Cu") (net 19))
 (segment (start 89.4 172.5) (end 90.5 173.6) (width 2.5) (layer "F.Cu") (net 19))
 (segment (start 113.105 169.105) (end 99.335 169.105) (width 2.5) (layer "F.Cu") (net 19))
 (segment (start 99.335 171.565) (end 99.335 169.105) (width 2.5) (layer "F.Cu") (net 19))
 (segment (start 89.4 168.2) (end 89.4 172.5) (width 2.5) (layer "F.Cu") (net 19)))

